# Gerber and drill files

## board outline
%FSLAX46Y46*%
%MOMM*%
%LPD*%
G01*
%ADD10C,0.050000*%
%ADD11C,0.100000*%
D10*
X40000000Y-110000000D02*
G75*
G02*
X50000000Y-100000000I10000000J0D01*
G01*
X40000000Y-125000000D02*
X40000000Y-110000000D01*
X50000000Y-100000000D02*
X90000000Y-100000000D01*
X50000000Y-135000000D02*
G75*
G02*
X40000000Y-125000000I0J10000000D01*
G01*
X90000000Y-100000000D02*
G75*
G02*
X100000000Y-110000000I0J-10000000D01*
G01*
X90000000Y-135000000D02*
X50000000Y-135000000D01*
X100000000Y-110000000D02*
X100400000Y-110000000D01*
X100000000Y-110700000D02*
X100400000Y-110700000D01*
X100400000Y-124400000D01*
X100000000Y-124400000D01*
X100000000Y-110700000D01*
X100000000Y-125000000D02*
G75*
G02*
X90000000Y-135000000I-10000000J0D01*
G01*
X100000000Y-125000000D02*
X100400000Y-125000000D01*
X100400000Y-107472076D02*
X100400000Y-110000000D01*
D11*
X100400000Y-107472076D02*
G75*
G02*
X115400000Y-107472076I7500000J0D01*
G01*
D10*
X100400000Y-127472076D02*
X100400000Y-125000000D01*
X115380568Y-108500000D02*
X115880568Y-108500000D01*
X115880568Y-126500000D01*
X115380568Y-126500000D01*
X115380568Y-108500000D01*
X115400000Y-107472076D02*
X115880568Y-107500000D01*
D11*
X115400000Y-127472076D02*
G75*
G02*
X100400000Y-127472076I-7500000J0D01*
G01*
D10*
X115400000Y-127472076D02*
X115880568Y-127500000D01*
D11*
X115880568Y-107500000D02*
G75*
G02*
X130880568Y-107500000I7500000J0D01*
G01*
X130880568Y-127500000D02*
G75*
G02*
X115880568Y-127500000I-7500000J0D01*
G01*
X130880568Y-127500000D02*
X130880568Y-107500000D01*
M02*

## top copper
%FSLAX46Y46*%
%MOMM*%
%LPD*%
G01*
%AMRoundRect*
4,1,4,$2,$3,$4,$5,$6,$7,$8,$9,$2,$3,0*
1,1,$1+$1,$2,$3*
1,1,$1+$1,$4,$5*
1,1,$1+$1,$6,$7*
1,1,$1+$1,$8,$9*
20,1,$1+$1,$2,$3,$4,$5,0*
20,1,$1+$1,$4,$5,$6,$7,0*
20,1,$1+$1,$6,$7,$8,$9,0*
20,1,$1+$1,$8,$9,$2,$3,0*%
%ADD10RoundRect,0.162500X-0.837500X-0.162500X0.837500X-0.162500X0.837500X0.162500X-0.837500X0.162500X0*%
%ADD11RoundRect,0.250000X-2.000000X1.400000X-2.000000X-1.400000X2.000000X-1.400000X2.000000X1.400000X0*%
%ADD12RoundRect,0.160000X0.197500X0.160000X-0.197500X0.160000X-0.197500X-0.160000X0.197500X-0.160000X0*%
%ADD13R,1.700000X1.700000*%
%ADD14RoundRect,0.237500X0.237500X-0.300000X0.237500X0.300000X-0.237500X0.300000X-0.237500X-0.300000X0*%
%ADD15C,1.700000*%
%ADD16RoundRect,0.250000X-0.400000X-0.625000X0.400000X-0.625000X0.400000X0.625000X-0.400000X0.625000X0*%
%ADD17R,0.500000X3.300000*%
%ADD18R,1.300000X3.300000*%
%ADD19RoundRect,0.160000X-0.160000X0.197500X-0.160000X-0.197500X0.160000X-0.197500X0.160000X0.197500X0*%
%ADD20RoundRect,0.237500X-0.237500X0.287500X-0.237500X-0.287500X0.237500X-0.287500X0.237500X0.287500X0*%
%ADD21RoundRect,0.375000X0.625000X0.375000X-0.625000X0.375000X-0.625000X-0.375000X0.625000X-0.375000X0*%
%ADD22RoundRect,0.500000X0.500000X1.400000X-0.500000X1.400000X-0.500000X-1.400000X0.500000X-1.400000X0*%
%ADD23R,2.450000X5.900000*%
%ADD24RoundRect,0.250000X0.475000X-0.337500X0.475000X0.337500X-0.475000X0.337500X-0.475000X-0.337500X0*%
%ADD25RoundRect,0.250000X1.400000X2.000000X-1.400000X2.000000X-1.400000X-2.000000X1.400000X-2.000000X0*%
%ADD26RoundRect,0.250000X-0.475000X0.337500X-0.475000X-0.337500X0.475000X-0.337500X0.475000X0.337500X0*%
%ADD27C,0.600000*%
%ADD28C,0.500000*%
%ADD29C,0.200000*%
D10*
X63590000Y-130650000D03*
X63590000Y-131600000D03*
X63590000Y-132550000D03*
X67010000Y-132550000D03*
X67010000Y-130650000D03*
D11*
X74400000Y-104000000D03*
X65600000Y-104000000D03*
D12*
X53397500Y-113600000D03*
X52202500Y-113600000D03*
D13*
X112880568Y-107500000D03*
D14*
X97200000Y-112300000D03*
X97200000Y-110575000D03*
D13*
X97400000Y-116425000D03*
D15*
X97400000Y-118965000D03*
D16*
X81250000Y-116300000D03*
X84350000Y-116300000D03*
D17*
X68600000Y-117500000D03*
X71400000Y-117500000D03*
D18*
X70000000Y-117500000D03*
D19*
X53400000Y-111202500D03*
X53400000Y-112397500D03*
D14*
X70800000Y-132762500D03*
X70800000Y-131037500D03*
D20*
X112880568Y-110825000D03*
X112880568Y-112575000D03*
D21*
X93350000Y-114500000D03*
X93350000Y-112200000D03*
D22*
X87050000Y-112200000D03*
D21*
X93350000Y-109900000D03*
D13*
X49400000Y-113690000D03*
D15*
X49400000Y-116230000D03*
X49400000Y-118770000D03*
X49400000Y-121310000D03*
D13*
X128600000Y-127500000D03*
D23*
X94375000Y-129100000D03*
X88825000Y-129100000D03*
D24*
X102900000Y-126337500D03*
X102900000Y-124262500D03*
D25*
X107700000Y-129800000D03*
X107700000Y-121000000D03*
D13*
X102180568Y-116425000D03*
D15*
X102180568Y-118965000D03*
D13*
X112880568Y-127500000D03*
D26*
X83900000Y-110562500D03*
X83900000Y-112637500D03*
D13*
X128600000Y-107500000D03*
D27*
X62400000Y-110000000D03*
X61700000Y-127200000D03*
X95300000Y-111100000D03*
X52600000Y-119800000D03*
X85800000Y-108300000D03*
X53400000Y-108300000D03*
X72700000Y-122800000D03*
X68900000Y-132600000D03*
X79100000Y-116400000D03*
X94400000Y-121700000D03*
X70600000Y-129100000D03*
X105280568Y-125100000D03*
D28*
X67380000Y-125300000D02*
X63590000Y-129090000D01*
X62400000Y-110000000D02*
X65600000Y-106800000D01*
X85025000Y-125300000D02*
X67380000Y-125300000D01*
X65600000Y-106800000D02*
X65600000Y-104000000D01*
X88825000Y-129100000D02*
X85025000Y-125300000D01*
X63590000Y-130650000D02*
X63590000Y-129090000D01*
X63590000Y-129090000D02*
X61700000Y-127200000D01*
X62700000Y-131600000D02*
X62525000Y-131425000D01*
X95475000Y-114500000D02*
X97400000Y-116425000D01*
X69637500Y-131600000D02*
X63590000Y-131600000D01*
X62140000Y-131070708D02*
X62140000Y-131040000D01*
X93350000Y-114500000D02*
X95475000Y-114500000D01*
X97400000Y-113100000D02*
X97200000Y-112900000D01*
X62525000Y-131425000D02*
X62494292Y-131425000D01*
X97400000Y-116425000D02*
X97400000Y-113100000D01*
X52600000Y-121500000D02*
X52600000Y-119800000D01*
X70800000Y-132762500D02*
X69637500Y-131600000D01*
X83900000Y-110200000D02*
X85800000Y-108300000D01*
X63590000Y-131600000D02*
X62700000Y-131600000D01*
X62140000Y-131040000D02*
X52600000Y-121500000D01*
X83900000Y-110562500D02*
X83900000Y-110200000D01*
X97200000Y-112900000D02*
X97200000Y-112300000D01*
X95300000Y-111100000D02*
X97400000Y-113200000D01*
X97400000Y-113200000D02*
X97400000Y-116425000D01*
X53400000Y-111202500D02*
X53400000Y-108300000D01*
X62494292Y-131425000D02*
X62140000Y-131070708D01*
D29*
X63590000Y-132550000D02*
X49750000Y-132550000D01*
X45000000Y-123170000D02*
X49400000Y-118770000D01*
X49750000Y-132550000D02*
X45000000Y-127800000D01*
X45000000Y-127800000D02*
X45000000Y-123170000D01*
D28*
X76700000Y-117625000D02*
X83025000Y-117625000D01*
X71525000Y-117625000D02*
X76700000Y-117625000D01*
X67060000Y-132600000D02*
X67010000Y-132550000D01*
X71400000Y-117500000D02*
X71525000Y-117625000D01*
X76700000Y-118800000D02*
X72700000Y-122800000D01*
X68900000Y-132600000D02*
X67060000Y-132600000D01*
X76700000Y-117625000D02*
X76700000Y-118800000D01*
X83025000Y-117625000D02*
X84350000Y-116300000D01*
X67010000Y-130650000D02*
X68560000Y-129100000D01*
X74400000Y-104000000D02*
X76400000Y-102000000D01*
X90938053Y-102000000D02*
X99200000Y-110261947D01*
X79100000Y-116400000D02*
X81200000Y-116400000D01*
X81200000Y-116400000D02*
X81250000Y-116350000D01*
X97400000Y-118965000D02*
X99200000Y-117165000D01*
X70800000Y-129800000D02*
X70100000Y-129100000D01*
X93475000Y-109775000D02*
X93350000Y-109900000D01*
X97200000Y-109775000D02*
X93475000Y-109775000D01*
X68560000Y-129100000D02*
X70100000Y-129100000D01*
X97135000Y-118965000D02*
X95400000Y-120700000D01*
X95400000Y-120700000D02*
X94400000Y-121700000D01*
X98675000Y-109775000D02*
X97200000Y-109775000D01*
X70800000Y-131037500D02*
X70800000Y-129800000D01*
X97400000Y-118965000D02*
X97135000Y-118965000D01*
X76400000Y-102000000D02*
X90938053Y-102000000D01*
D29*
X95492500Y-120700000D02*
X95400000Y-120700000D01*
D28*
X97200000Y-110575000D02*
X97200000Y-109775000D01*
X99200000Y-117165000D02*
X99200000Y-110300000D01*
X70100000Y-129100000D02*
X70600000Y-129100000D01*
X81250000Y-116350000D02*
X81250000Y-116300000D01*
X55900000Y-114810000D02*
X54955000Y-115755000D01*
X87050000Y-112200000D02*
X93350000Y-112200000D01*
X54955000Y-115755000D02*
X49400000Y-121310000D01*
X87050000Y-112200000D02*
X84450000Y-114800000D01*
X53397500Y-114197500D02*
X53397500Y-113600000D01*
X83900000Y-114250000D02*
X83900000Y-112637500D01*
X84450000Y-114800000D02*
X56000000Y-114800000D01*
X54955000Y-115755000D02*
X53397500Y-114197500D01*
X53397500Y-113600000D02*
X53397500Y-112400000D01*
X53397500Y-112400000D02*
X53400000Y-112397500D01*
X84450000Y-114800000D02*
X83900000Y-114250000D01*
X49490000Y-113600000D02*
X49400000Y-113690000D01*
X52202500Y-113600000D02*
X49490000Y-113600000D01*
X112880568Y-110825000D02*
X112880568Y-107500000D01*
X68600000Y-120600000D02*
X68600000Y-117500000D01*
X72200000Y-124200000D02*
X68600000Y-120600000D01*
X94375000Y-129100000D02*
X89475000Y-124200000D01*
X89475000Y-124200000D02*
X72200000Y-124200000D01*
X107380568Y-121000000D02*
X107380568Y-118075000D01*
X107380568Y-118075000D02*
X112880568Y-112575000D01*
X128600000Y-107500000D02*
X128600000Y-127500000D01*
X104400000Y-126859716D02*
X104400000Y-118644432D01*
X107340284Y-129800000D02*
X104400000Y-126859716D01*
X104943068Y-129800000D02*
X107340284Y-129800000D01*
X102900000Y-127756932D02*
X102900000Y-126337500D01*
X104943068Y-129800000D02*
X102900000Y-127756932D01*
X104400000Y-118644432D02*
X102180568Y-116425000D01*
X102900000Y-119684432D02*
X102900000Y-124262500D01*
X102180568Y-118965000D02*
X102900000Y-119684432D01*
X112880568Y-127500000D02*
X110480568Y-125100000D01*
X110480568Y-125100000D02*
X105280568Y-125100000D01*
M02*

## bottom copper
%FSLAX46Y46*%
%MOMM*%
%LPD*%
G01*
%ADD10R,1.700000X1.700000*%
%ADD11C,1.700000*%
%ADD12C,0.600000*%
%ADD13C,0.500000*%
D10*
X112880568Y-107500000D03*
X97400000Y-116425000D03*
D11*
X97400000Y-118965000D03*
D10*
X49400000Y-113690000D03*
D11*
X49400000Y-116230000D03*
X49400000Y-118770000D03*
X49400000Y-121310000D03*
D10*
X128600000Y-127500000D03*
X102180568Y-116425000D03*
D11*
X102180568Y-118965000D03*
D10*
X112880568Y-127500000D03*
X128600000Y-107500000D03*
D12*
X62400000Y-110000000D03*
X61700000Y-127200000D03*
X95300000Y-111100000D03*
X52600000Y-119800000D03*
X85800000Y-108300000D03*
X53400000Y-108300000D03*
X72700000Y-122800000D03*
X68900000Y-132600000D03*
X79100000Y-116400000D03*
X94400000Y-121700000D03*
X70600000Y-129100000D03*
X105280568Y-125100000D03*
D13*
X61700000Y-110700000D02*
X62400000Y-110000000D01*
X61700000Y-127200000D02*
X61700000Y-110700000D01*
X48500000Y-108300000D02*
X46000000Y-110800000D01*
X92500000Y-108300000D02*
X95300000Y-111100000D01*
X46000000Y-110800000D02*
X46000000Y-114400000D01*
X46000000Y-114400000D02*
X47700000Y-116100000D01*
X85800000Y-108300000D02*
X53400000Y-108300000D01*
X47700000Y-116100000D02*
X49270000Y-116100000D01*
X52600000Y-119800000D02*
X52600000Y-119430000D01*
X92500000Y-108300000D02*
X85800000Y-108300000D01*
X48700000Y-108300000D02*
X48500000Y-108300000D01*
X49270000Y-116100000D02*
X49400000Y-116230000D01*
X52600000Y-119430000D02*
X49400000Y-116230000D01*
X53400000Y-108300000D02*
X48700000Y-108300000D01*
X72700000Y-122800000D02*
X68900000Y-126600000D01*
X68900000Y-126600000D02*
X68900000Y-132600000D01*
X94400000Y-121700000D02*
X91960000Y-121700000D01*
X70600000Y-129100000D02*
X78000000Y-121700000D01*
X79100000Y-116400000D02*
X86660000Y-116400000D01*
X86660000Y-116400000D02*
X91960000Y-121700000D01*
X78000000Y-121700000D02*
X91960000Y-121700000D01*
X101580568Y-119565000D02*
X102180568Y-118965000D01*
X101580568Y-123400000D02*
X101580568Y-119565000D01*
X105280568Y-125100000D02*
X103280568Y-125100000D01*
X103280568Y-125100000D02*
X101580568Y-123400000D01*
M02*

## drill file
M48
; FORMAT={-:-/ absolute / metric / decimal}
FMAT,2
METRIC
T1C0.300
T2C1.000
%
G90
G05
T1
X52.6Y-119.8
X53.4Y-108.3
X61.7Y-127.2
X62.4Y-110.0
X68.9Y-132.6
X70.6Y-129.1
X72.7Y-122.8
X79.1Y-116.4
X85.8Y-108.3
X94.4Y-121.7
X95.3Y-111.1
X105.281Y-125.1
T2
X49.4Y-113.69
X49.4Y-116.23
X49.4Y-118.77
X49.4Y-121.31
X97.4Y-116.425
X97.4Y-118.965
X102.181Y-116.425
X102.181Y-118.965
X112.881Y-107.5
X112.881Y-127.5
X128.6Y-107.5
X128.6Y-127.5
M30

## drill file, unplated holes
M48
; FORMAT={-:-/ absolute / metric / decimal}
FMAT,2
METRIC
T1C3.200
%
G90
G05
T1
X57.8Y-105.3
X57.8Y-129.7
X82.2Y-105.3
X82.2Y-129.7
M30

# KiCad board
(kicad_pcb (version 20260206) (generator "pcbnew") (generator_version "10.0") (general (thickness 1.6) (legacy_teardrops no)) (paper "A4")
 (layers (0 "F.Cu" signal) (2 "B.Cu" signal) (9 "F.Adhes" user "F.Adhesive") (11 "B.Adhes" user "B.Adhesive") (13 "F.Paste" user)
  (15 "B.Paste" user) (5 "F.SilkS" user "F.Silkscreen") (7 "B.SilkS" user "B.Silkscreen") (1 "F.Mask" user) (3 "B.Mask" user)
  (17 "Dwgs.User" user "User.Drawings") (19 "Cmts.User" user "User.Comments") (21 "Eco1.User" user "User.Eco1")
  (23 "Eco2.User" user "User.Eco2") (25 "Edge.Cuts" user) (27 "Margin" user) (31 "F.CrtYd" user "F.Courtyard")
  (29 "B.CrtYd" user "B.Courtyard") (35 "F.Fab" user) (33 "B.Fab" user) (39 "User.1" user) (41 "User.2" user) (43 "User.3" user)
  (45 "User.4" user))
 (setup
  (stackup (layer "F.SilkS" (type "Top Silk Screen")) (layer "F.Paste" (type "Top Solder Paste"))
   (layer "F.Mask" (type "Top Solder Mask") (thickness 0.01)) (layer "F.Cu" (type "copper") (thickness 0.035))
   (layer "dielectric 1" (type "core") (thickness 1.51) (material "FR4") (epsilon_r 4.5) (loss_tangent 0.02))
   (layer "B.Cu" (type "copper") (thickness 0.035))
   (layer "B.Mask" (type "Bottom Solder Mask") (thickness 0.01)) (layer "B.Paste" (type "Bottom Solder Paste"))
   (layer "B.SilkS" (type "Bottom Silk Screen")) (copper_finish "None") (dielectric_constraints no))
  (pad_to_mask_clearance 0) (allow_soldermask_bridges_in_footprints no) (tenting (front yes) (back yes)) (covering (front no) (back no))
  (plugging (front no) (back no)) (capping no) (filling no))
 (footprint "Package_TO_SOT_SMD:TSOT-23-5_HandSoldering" (layer "F.Cu") (at 65.3 131.6)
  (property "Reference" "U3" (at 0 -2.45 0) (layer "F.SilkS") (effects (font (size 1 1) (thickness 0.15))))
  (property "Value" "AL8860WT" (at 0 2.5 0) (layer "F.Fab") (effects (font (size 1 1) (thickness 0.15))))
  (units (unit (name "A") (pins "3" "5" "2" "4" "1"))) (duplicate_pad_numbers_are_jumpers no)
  (pad "1" smd roundrect (at -1.71 -0.95) (size 2 0.65) (layers "F.Cu" "F.Mask" "F.Paste") (roundrect_rratio 0.25) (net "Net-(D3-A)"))
  (pad "2" smd roundrect (at -1.71 0) (size 2 0.65) (layers "F.Cu" "F.Mask" "F.Paste") (roundrect_rratio 0.25) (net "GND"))
  (pad "3" smd roundrect (at -1.71 0.95) (size 2 0.65) (layers "F.Cu" "F.Mask" "F.Paste") (roundrect_rratio 0.25) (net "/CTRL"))
  (pad "4" smd roundrect (at 1.71 0.95) (size 2 0.65) (layers "F.Cu" "F.Mask" "F.Paste") (roundrect_rratio 0.25) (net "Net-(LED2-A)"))
  (pad "5" smd roundrect (at 1.71 -0.95) (size 2 0.65) (layers "F.Cu" "F.Mask" "F.Paste") (roundrect_rratio 0.25) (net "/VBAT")))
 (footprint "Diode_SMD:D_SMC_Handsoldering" (layer "F.Cu") (at 70 104 180)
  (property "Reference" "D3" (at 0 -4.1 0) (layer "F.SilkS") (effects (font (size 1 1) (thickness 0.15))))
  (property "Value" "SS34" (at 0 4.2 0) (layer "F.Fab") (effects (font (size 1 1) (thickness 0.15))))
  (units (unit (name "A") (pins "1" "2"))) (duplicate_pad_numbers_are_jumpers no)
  (pad "1" smd roundrect (at -4.4 0 270) (size 3.3 4.5) (layers "F.Cu" "F.Mask" "F.Paste") (roundrect_rratio 0.0757575758) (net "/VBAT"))
  (pad "2" smd roundrect (at 4.4 0 270) (size 3.3 4.5) (layers "F.Cu" "F.Mask" "F.Paste") (roundrect_rratio 0.0757575758) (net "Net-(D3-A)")))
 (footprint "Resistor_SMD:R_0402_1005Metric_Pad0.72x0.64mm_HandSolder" (layer "F.Cu") (at 52.8 113.6 180)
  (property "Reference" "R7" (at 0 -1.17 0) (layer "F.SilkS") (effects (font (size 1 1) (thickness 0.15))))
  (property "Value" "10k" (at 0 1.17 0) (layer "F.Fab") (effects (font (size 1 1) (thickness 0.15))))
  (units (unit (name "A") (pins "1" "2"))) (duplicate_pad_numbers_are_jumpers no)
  (pad "1" smd roundrect (at -0.5975 0 180) (size 0.715 0.64) (layers "F.Cu" "F.Mask" "F.Paste") (roundrect_rratio 0.25) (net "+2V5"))
  (pad "2" smd roundrect (at 0.5975 0 180) (size 0.715 0.64) (layers "F.Cu" "F.Mask" "F.Paste") (roundrect_rratio 0.25)
   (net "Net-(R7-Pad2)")))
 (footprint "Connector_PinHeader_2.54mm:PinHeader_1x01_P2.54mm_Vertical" (layer "F.Cu") (at 112.880568 107.5)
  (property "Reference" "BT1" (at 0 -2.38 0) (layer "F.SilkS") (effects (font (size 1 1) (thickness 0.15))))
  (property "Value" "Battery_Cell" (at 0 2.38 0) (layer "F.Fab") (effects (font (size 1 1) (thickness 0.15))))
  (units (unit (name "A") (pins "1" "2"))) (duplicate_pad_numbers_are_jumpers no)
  (pad "1" thru_hole rect (at 0 0) (size 1.7 1.7) (drill 1) (layers "*.Cu" "*.Mask") (remove_unused_layers no) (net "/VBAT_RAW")))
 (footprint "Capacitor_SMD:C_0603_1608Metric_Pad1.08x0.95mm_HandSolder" (layer "F.Cu") (at 97.2 111.4375 90)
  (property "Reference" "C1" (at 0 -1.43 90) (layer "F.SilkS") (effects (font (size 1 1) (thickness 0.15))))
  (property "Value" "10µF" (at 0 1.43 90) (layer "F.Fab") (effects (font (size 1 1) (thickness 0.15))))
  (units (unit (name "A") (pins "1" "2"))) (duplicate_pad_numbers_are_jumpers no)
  (pad "1" smd roundrect (at -0.8625 0 90) (size 1.075 0.95) (layers "F.Cu" "F.Mask" "F.Paste") (roundrect_rratio 0.25) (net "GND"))
  (pad "2" smd roundrect (at 0.8625 0 90) (size 1.075 0.95) (layers "F.Cu" "F.Mask" "F.Paste") (roundrect_rratio 0.25) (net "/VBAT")))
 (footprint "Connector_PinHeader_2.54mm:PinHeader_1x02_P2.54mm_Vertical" (layer "F.Cu") (at 97.4 116.425)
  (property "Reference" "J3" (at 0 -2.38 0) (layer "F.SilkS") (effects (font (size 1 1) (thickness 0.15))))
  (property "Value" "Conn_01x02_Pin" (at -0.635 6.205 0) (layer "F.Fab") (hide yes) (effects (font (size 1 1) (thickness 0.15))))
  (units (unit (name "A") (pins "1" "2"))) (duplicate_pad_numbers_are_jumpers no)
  (pad "1" thru_hole rect (at 0 0) (size 1.7 1.7) (drill 1) (layers "*.Cu" "*.Mask") (remove_unused_layers no) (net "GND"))
  (pad "2" thru_hole circle (at 0 2.54) (size 1.7 1.7) (drill 1) (layers "*.Cu" "*.Mask") (remove_unused_layers no) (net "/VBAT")))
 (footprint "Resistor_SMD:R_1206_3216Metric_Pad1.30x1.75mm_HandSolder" (layer "F.Cu") (at 82.8 116.3)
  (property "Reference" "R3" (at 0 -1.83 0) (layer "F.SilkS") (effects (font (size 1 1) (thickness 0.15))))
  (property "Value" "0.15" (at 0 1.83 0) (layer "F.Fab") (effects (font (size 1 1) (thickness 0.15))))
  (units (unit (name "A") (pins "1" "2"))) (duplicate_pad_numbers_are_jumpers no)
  (pad "1" smd roundrect (at -1.55 0) (size 1.3 1.75) (layers "F.Cu" "F.Mask" "F.Paste") (roundrect_rratio 0.192308) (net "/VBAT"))
  (pad "2" smd roundrect (at 1.55 0) (size 1.3 1.75) (layers "F.Cu" "F.Mask" "F.Paste") (roundrect_rratio 0.192308) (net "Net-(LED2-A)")))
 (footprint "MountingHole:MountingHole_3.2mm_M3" (layer "F.Cu") (at 82.2 129.7)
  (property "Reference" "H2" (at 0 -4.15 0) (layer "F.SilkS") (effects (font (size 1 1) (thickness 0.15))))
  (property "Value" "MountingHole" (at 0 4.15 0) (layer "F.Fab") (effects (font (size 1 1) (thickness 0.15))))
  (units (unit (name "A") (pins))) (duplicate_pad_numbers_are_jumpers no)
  (pad "" np_thru_hole circle (at 0 0) (size 3.2 3.2) (drill 3.2) (layers "*.Cu" "*.Mask")))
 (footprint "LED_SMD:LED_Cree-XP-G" (layer "F.Cu") (at 70 117.5)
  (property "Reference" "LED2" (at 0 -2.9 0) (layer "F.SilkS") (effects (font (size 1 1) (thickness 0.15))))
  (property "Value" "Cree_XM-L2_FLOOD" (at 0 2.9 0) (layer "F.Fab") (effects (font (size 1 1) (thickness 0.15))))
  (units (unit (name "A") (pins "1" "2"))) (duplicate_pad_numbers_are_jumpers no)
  (pad "" smd rect (at 0 -1) (size 1.01 0.75) (layers "F.Paste"))
  (pad "" smd rect (at 0 0) (size 1.01 0.75) (layers "F.Paste"))
  (pad "" smd rect (at 0 1) (size 1.01 0.75) (layers "F.Paste"))
  (pad "1" smd rect (at -1.4 0) (size 0.5 3.3) (layers "F.Cu" "F.Mask" "F.Paste") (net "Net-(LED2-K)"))
  (pad "2" smd rect (at 1.4 0) (size 0.5 3.3) (layers "F.Cu" "F.Mask" "F.Paste") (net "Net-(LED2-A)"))
  (pad "3" smd rect (at 0 0) (size 1.3 3.3) (layers "F.Cu" "F.Mask")))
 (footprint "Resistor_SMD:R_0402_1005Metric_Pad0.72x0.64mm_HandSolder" (layer "F.Cu") (at 53.4 111.8 -90)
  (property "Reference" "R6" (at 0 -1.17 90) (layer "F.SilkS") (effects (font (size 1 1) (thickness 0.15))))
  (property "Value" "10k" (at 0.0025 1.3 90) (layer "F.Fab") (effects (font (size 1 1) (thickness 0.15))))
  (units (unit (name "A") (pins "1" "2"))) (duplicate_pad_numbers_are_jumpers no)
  (pad "1" smd roundrect (at -0.5975 0 270) (size 0.715 0.64) (layers "F.Cu" "F.Mask" "F.Paste") (roundrect_rratio 0.25) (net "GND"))
  (pad "2" smd roundrect (at 0.5975 0 270) (size 0.715 0.64) (layers "F.Cu" "F.Mask" "F.Paste") (roundrect_rratio 0.25) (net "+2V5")))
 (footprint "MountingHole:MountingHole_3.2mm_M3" (layer "F.Cu") (at 57.8 129.7)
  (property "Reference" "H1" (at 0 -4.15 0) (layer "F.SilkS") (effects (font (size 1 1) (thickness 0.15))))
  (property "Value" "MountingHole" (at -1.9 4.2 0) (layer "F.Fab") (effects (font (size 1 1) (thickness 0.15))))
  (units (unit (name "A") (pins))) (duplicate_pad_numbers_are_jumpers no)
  (pad "" np_thru_hole circle (at 0 0) (size 3.2 3.2) (drill 3.2) (layers "*.Cu" "*.Mask")))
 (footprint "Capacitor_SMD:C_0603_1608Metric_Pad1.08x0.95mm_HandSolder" (layer "F.Cu") (at 70.8 131.9 90)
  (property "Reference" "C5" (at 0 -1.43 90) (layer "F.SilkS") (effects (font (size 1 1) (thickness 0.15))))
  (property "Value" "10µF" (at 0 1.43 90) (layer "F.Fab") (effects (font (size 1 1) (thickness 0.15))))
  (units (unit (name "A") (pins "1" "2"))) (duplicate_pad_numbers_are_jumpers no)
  (pad "1" smd roundrect (at -0.8625 0 90) (size 1.075 0.95) (layers "F.Cu" "F.Mask" "F.Paste") (roundrect_rratio 0.25) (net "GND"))
  (pad "2" smd roundrect (at 0.8625 0 90) (size 1.075 0.95) (layers "F.Cu" "F.Mask" "F.Paste") (roundrect_rratio 0.25) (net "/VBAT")))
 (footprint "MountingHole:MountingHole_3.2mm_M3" (layer "F.Cu") (at 57.8 105.3)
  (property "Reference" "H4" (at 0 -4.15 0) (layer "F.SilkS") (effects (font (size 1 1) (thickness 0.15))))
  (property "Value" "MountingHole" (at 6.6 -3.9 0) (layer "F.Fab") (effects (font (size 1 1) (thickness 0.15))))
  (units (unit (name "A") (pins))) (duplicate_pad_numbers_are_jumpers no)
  (pad "" np_thru_hole circle (at 0 0) (size 3.2 3.2) (drill 3.2) (layers "*.Cu" "*.Mask")))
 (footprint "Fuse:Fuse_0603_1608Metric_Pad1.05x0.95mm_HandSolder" (layer "F.Cu") (at 112.880568 111.7 -90)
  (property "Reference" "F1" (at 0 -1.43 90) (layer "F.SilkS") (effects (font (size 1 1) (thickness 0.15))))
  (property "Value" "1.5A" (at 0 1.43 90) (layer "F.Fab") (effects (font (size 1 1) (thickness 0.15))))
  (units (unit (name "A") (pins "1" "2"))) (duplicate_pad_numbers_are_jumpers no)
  (pad "1" smd roundrect (at -0.875 0 270) (size 1.05 0.95) (layers "F.Cu" "F.Mask" "F.Paste") (roundrect_rratio 0.25) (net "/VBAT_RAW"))
  (pad "2" smd roundrect (at 0.875 0 270) (size 1.05 0.95) (layers "F.Cu" "F.Mask" "F.Paste") (roundrect_rratio 0.25) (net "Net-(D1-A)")))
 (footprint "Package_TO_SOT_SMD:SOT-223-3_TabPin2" (layer "F.Cu") (at 90.2 112.2 180)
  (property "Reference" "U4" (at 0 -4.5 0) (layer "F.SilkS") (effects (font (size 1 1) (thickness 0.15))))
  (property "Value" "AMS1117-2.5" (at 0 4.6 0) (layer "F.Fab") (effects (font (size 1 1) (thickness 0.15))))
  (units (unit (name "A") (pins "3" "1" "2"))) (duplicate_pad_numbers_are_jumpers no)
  (pad "1" smd roundrect (at -3.15 -2.3 180) (size 2 1.5) (layers "F.Cu" "F.Mask" "F.Paste") (roundrect_rratio 0.25) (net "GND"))
  (pad "2" smd roundrect (at -3.15 0 180) (size 2 1.5) (layers "F.Cu" "F.Mask" "F.Paste") (roundrect_rratio 0.25) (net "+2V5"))
  (pad "2" smd roundrect (at 3.15 0 180) (size 2 3.8) (layers "F.Cu" "F.Mask" "F.Paste") (roundrect_rratio 0.25) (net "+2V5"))
  (pad "3" smd roundrect (at -3.15 2.3 180) (size 2 1.5) (layers "F.Cu" "F.Mask" "F.Paste") (roundrect_rratio 0.25) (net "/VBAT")))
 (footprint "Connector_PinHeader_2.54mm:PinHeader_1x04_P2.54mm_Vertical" (layer "F.Cu") (at 49.4 113.69)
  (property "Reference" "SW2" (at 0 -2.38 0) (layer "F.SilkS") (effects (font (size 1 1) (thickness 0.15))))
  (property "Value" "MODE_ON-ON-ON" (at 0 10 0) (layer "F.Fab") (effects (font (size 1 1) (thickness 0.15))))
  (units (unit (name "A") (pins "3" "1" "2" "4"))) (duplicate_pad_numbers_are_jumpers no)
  (pad "1" thru_hole rect (at 0 0) (size 1.7 1.7) (drill 1) (layers "*.Cu" "*.Mask") (remove_unused_layers no) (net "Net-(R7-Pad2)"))
  (pad "2" thru_hole circle (at 0 2.54) (size 1.7 1.7) (drill 1) (layers "*.Cu" "*.Mask") (remove_unused_layers no) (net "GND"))
  (pad "3" thru_hole circle (at 0 5.08) (size 1.7 1.7) (drill 1) (layers "*.Cu" "*.Mask") (remove_unused_layers no) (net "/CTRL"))
  (pad "4" thru_hole circle (at 0 7.62) (size 1.7 1.7) (drill 1) (layers "*.Cu" "*.Mask") (remove_unused_layers no) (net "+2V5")))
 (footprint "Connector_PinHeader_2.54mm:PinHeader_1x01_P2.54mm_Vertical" (layer "F.Cu") (at 128.6 127.5)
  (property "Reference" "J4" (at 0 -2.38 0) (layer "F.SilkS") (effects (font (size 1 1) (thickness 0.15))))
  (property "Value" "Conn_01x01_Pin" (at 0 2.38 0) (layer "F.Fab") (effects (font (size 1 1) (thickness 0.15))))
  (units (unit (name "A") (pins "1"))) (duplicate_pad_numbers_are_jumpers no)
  (pad "1" thru_hole rect (at 0 0) (size 1.7 1.7) (drill 1) (layers "*.Cu" "*.Mask") (remove_unused_layers no) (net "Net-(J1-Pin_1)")))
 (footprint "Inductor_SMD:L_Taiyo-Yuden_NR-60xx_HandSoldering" (layer "F.Cu") (at 91.6 129.1 180)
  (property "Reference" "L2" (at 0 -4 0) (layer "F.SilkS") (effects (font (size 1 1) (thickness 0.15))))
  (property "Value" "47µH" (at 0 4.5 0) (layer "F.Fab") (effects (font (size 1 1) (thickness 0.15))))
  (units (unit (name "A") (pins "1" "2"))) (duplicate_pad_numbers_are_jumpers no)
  (pad "1" smd rect (at -2.775 0 180) (size 2.45 5.9) (layers "F.Cu" "F.Mask" "F.Paste") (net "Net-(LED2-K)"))
  (pad "2" smd rect (at 2.775 0 180) (size 2.45 5.9) (layers "F.Cu" "F.Mask" "F.Paste") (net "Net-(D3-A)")))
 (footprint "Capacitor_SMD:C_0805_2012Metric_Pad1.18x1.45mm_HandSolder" (layer "F.Cu") (at 102.9 125.3 90)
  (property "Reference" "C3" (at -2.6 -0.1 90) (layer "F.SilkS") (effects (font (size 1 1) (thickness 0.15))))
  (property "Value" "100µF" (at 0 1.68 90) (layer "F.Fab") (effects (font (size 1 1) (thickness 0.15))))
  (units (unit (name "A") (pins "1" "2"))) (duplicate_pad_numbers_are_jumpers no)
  (pad "1" smd roundrect (at -1.0375 0 90) (size 1.175 1.45) (layers "F.Cu" "F.Mask" "F.Paste") (roundrect_rratio 0.212766)
   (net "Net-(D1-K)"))
  (pad "2" smd roundrect (at 1.0375 0 90) (size 1.175 1.45) (layers "F.Cu" "F.Mask" "F.Paste") (roundrect_rratio 0.212766) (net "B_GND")))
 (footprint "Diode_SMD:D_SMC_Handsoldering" (layer "F.Cu") (at 107.7 125.4 90)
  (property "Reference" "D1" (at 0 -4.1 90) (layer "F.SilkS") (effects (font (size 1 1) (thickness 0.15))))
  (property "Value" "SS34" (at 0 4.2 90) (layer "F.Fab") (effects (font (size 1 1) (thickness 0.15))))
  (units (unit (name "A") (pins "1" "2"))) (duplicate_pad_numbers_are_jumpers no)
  (pad "1" smd roundrect (at -4.4 0 180) (size 3.3 4.5) (layers "F.Cu" "F.Mask" "F.Paste") (roundrect_rratio 0.0757575758)
   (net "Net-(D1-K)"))
  (pad "2" smd roundrect (at 4.4 0 180) (size 3.3 4.5) (layers "F.Cu" "F.Mask" "F.Paste") (roundrect_rratio 0.0757575758) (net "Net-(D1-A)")))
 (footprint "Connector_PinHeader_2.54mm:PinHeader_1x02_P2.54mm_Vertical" (layer "F.Cu") (at 102.180568 116.425)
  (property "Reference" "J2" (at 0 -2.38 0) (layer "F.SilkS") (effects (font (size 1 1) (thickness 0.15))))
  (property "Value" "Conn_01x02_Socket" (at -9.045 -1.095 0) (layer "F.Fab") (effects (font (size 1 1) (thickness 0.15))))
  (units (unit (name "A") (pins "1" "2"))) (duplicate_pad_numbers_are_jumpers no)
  (pad "1" thru_hole rect (at 0 0) (size 1.7 1.7) (drill 1) (layers "*.Cu" "*.Mask") (remove_unused_layers no) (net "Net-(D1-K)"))
  (pad "2" thru_hole circle (at 0 2.54) (size 1.7 1.7) (drill 1) (layers "*.Cu" "*.Mask") (remove_unused_layers no) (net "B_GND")))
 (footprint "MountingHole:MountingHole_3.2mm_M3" (layer "F.Cu") (at 82.2 105.3)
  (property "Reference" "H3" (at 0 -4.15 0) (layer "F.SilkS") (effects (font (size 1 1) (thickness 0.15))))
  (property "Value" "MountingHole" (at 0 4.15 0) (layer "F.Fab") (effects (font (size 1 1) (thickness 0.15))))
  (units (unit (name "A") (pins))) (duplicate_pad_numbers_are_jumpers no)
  (pad "" np_thru_hole circle (at 0 0) (size 3.2 3.2) (drill 3.2) (layers "*.Cu" "*.Mask")))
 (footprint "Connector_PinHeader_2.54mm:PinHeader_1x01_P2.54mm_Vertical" (layer "F.Cu") (at 112.880568 127.5)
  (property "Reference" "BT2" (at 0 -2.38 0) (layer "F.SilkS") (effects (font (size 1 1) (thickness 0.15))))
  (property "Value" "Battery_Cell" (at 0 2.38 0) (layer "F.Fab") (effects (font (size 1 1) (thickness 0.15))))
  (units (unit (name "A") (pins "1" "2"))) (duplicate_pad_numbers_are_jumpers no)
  (pad "1" thru_hole rect (at 0 0) (size 1.7 1.7) (drill 1) (layers "*.Cu" "*.Mask") (remove_unused_layers no) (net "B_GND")))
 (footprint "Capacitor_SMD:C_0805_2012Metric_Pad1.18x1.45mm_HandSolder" (layer "F.Cu") (at 83.9 111.6 -90)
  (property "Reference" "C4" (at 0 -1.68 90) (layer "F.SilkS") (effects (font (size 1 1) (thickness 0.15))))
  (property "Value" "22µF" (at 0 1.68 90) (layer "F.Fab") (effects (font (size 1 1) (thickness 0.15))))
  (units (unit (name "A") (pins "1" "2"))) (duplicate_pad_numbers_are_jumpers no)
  (pad "1" smd roundrect (at -1.0375 0 270) (size 1.175 1.45) (layers "F.Cu" "F.Mask" "F.Paste") (roundrect_rratio 0.212766) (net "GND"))
  (pad "2" smd roundrect (at 1.0375 0 270) (size 1.175 1.45) (layers "F.Cu" "F.Mask" "F.Paste") (roundrect_rratio 0.212766) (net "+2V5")))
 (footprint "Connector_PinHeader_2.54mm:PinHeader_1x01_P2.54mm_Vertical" (layer "F.Cu") (at 128.6 107.5)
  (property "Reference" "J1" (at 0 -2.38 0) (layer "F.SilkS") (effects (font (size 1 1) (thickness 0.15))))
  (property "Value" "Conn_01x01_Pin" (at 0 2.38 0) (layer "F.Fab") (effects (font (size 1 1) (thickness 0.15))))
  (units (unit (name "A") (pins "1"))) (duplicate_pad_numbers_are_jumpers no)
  (pad "1" thru_hole rect (at 0 0) (size 1.7 1.7) (drill 1) (layers "*.Cu" "*.Mask") (remove_unused_layers no) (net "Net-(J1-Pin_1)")))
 (gr_arc (start 40 110) (mid 42.928932 102.928932) (end 50 100) (stroke (width 0.05) (type default)) (layer "Edge.Cuts"))
 (gr_line (start 40 125) (end 40 110) (stroke (width 0.05) (type default)) (layer "Edge.Cuts"))
 (gr_line (start 50 100) (end 90 100) (stroke (width 0.05) (type default)) (layer "Edge.Cuts"))
 (gr_arc (start 50 135) (mid 42.928932 132.071068) (end 40 125) (stroke (width 0.05) (type default)) (layer "Edge.Cuts"))
 (gr_arc (start 90 100) (mid 97.071068 102.928932) (end 100 110) (stroke (width 0.05) (type default)) (layer "Edge.Cuts"))
 (gr_line (start 90 135) (end 50 135) (stroke (width 0.05) (type default)) (layer "Edge.Cuts"))
 (gr_line (start 100 110) (end 100.4 110) (stroke (width 0.05) (type default)) (layer "Edge.Cuts"))
 (gr_rect (start 100 110.7) (end 100.4 124.4) (stroke (width 0.05) (type default)) (fill no) (layer "Edge.Cuts"))
 (gr_arc (start 100 125) (mid 97.071068 132.071068) (end 90 135) (stroke (width 0.05) (type default)) (layer "Edge.Cuts"))
 (gr_line (start 100 125) (end 100.4 125) (stroke (width 0.05) (type default)) (layer "Edge.Cuts"))
 (gr_line (start 100.4 107.472076) (end 100.4 110) (stroke (width 0.05) (type default)) (layer "Edge.Cuts"))
 (gr_arc (start 100.4 107.472076) (mid 107.9 99.972076) (end 115.4 107.472076) (stroke (width 0.1) (type solid)) (layer "Edge.Cuts"))
 (gr_line (start 100.4 127.472076) (end 100.4 125) (stroke (width 0.05) (type default)) (layer "Edge.Cuts"))
 (gr_rect (start 115.380568 108.5) (end 115.880568 126.5) (stroke (width 0.05) (type default)) (fill no) (layer "Edge.Cuts"))
 (gr_line (start 115.4 107.472076) (end 115.880568 107.5) (stroke (width 0.05) (type default)) (layer "Edge.Cuts"))
 (gr_arc (start 115.4 127.472076) (mid 107.9 134.972076) (end 100.4 127.472076) (stroke (width 0.1) (type solid)) (layer "Edge.Cuts"))
 (gr_line (start 115.4 127.472076) (end 115.880568 127.5) (stroke (width 0.05) (type default)) (layer "Edge.Cuts"))
 (gr_arc (start 115.880568 107.5) (mid 123.380568 100) (end 130.880568 107.5) (stroke (width 0.1) (type solid)) (layer "Edge.Cuts"))
 (gr_arc (start 130.880568 127.5) (mid 123.380568 135) (end 115.880568 127.5) (stroke (width 0.1) (type solid)) (layer "Edge.Cuts"))
 (gr_line (start 130.880568 127.5) (end 130.880568 107.5) (stroke (width 0.1) (type solid)) (layer "Edge.Cuts"))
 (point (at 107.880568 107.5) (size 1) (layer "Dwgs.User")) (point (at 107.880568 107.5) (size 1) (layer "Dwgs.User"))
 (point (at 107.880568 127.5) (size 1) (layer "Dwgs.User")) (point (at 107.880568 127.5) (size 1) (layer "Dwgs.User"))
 (segment (start 67.38 125.3) (end 63.59 129.09) (width 0.5) (layer "F.Cu") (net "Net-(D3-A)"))
 (segment (start 62.4 110) (end 65.6 106.8) (width 0.5) (layer "F.Cu") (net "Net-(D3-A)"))
 (segment (start 85.025 125.3) (end 67.38 125.3) (width 0.5) (layer "F.Cu") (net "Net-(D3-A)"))
 (segment (start 65.6 106.8) (end 65.6 104) (width 0.5) (layer "F.Cu") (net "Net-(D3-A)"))
 (segment (start 88.825 129.1) (end 85.025 125.3) (width 0.5) (layer "F.Cu") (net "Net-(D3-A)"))
 (segment (start 63.59 130.65) (end 63.59 129.09) (width 0.5) (layer "F.Cu") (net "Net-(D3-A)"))
 (segment (start 63.59 129.09) (end 61.7 127.2) (width 0.5) (layer "F.Cu") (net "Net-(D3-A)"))
 (via (at 62.4 110) (size 0.6) (drill 0.3) (layers "F.Cu" "B.Cu") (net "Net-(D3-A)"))
 (via (at 61.7 127.2) (size 0.6) (drill 0.3) (layers "F.Cu" "B.Cu") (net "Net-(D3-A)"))
 (segment (start 61.7 110.7) (end 62.4 110) (width 0.5) (layer "B.Cu") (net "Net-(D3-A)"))
 (segment (start 61.7 127.2) (end 61.7 110.7) (width 0.5) (layer "B.Cu") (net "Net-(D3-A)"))
 (segment (start 62.7 131.6) (end 62.525 131.425) (width 0.5) (layer "F.Cu") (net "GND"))
 (segment (start 95.475 114.5) (end 97.4 116.425) (width 0.5) (layer "F.Cu") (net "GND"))
 (segment (start 69.6375 131.6) (end 63.59 131.6) (width 0.5) (layer "F.Cu") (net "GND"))
 (segment (start 62.14 131.070708) (end 62.14 131.04) (width 0.5) (layer "F.Cu") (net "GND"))
 (segment (start 93.35 114.5) (end 95.475 114.5) (width 0.5) (layer "F.Cu") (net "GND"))
 (segment (start 97.4 113.1) (end 97.2 112.9) (width 0.5) (layer "F.Cu") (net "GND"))
 (segment (start 62.525 131.425) (end 62.494292 131.425) (width 0.5) (layer "F.Cu") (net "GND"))
 (segment (start 97.4 116.425) (end 97.4 113.1) (width 0.5) (layer "F.Cu") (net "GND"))
 (segment (start 52.6 121.5) (end 52.6 119.8) (width 0.5) (layer "F.Cu") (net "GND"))
 (segment (start 70.8 132.7625) (end 69.6375 131.6) (width 0.5) (layer "F.Cu") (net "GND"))
 (segment (start 83.9 110.2) (end 85.8 108.3) (width 0.5) (layer "F.Cu") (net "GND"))
 (segment (start 63.59 131.6) (end 62.7 131.6) (width 0.5) (layer "F.Cu") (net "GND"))
 (segment (start 62.14 131.04) (end 52.6 121.5) (width 0.5) (layer "F.Cu") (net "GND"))
 (segment (start 83.9 110.5625) (end 83.9 110.2) (width 0.5) (layer "F.Cu") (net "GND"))
 (segment (start 97.2 112.9) (end 97.2 112.3) (width 0.5) (layer "F.Cu") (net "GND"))
 (segment (start 95.3 111.1) (end 97.4 113.2) (width 0.5) (layer "F.Cu") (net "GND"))
 (segment (start 97.4 113.2) (end 97.4 116.425) (width 0.5) (layer "F.Cu") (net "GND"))
 (segment (start 53.4 111.2025) (end 53.4 108.3) (width 0.5) (layer "F.Cu") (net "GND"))
 (segment (start 62.494292 131.425) (end 62.14 131.070708) (width 0.5) (layer "F.Cu") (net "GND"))
 (via (at 95.3 111.1) (size 0.6) (drill 0.3) (layers "F.Cu" "B.Cu") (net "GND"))
 (via (at 52.6 119.8) (size 0.6) (drill 0.3) (layers "F.Cu" "B.Cu") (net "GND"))
 (via (at 85.8 108.3) (size 0.6) (drill 0.3) (layers "F.Cu" "B.Cu") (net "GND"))
 (via (at 53.4 108.3) (size 0.6) (drill 0.3) (layers "F.Cu" "B.Cu") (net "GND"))
 (segment (start 48.5 108.3) (end 46 110.8) (width 0.5) (layer "B.Cu") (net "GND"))
 (segment (start 92.5 108.3) (end 95.3 111.1) (width 0.5) (layer "B.Cu") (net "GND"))
 (segment (start 46 110.8) (end 46 114.4) (width 0.5) (layer "B.Cu") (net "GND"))
 (segment (start 46 114.4) (end 47.7 116.1) (width 0.5) (layer "B.Cu") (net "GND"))
 (segment (start 85.8 108.3) (end 53.4 108.3) (width 0.5) (layer "B.Cu") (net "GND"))
 (segment (start 47.7 116.1) (end 49.27 116.1) (width 0.5) (layer "B.Cu") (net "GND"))
 (segment (start 52.6 119.8) (end 52.6 119.43) (width 0.5) (layer "B.Cu") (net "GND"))
 (segment (start 92.5 108.3) (end 85.8 108.3) (width 0.5) (layer "B.Cu") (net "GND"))
 (segment (start 48.7 108.3) (end 48.5 108.3) (width 0.5) (layer "B.Cu") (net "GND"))
 (segment (start 49.27 116.1) (end 49.4 116.23) (width 0.5) (layer "B.Cu") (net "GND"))
 (segment (start 52.6 119.43) (end 49.4 116.23) (width 0.5) (layer "B.Cu") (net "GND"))
 (segment (start 53.4 108.3) (end 48.7 108.3) (width 0.5) (layer "B.Cu") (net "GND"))
 (segment (start 63.59 132.55) (end 49.75 132.55) (width 0.2) (layer "F.Cu") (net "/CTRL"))
 (segment (start 45 123.17) (end 49.4 118.77) (width 0.2) (layer "F.Cu") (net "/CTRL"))
 (segment (start 49.75 132.55) (end 45 127.8) (width 0.2) (layer "F.Cu") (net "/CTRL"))
 (segment (start 45 127.8) (end 45 123.17) (width 0.2) (layer "F.Cu") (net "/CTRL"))
 (segment (start 76.7 117.625) (end 83.025 117.625) (width 0.5) (layer "F.Cu") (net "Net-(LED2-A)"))
 (segment (start 71.525 117.625) (end 76.7 117.625) (width 0.5) (layer "F.Cu") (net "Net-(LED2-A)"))
 (segment (start 67.06 132.6) (end 67.01 132.55) (width 0.5) (layer "F.Cu") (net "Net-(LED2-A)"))
 (segment (start 71.4 117.5) (end 71.525 117.625) (width 0.5) (layer "F.Cu") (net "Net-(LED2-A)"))
 (segment (start 76.7 118.8) (end 72.7 122.8) (width 0.5) (layer "F.Cu") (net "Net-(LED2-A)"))
 (segment (start 68.9 132.6) (end 67.06 132.6) (width 0.5) (layer "F.Cu") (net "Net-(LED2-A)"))
 (segment (start 76.7 117.625) (end 76.7 118.8) (width 0.5) (layer "F.Cu") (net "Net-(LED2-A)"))
 (segment (start 83.025 117.625) (end 84.35 116.3) (width 0.5) (layer "F.Cu") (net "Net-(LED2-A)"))
 (via (at 72.7 122.8) (size 0.6) (drill 0.3) (layers "F.Cu" "B.Cu") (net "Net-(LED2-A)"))
 (via (at 68.9 132.6) (size 0.6) (drill 0.3) (layers "F.Cu" "B.Cu") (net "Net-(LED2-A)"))
 (segment (start 72.7 122.8) (end 68.9 126.6) (width 0.5) (layer "B.Cu") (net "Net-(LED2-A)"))
 (segment (start 68.9 126.6) (end 68.9 132.6) (width 0.5) (layer "B.Cu") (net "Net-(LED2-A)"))
 (segment (start 67.01 130.65) (end 68.56 129.1) (width 0.5) (layer "F.Cu") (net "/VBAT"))
 (segment (start 74.4 104) (end 76.4 102) (width 0.5) (layer "F.Cu") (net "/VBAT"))
 (segment (start 90.938053 102) (end 99.2 110.261947) (width 0.5) (layer "F.Cu") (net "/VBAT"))
 (segment (start 79.1 116.4) (end 81.2 116.4) (width 0.5) (layer "F.Cu") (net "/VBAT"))
 (segment (start 81.2 116.4) (end 81.25 116.35) (width 0.5) (layer "F.Cu") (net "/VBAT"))
 (segment (start 97.4 118.965) (end 99.2 117.165) (width 0.5) (layer "F.Cu") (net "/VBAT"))
 (segment (start 70.8 129.8) (end 70.1 129.1) (width 0.5) (layer "F.Cu") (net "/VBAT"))
 (segment (start 93.475 109.775) (end 93.35 109.9) (width 0.5) (layer "F.Cu") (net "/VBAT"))
 (segment (start 97.2 109.775) (end 93.475 109.775) (width 0.5) (layer "F.Cu") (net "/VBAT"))
 (segment (start 68.56 129.1) (end 70.1 129.1) (width 0.5) (layer "F.Cu") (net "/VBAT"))
 (segment (start 97.135 118.965) (end 95.4 120.7) (width 0.5) (layer "F.Cu") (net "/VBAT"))
 (segment (start 95.4 120.7) (end 94.4 121.7) (width 0.5) (layer "F.Cu") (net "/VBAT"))
 (segment (start 98.675 109.775) (end 97.2 109.775) (width 0.5) (layer "F.Cu") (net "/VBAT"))
 (segment (start 70.8 131.0375) (end 70.8 129.8) (width 0.5) (layer "F.Cu") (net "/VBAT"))
 (segment (start 97.4 118.965) (end 97.135 118.965) (width 0.5) (layer "F.Cu") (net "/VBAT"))
 (segment (start 76.4 102) (end 90.938053 102) (width 0.5) (layer "F.Cu") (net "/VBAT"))
 (segment (start 95.4925 120.7) (end 95.4 120.7) (width 0.2) (layer "F.Cu") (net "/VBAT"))
 (segment (start 97.2 110.575) (end 97.2 109.775) (width 0.5) (layer "F.Cu") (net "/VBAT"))
 (segment (start 99.2 117.165) (end 99.2 110.3) (width 0.5) (layer "F.Cu") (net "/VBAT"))
 (segment (start 70.1 129.1) (end 70.6 129.1) (width 0.5) (layer "F.Cu") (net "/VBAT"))
 (segment (start 81.25 116.35) (end 81.25 116.3) (width 0.5) (layer "F.Cu") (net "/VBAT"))
 (via (at 79.1 116.4) (size 0.6) (drill 0.3) (layers "F.Cu" "B.Cu") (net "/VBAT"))
 (via (at 94.4 121.7) (size 0.6) (drill 0.3) (layers "F.Cu" "B.Cu") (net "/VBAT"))
 (via (at 70.6 129.1) (size 0.6) (drill 0.3) (layers "F.Cu" "B.Cu") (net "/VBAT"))
 (segment (start 94.4 121.7) (end 91.96 121.7) (width 0.5) (layer "B.Cu") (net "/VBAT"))
 (segment (start 70.6 129.1) (end 78 121.7) (width 0.5) (layer "B.Cu") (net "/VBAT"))
 (segment (start 79.1 116.4) (end 86.66 116.4) (width 0.5) (layer "B.Cu") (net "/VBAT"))
 (segment (start 86.66 116.4) (end 91.96 121.7) (width 0.5) (layer "B.Cu") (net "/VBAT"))
 (segment (start 78 121.7) (end 91.96 121.7) (width 0.5) (layer "B.Cu") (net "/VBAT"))
 (segment (start 55.9 114.81) (end 54.955 115.755) (width 0.5) (layer "F.Cu") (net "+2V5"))
 (segment (start 87.05 112.2) (end 93.35 112.2) (width 0.5) (layer "F.Cu") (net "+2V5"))
 (segment (start 54.955 115.755) (end 49.4 121.31) (width 0.5) (layer "F.Cu") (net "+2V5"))
 (segment (start 87.05 112.2) (end 84.45 114.8) (width 0.5) (layer "F.Cu") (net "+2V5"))
 (segment (start 53.3975 114.1975) (end 53.3975 113.6) (width 0.5) (layer "F.Cu") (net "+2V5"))
 (segment (start 83.9 114.25) (end 83.9 112.6375) (width 0.5) (layer "F.Cu") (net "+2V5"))
 (segment (start 84.45 114.8) (end 56 114.8) (width 0.5) (layer "F.Cu") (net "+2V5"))
 (segment (start 54.955 115.755) (end 53.3975 114.1975) (width 0.5) (layer "F.Cu") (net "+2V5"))
 (segment (start 53.3975 113.6) (end 53.3975 112.4) (width 0.5) (layer "F.Cu") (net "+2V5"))
 (segment (start 53.3975 112.4) (end 53.4 112.3975) (width 0.5) (layer "F.Cu") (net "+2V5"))
 (segment (start 84.45 114.8) (end 83.9 114.25) (width 0.5) (layer "F.Cu") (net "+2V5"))
 (segment (start 49.49 113.6) (end 49.4 113.69) (width 0.5) (layer "F.Cu") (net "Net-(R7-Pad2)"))
 (segment (start 52.2025 113.6) (end 49.49 113.6) (width 0.5) (layer "F.Cu") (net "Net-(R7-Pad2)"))
 (segment (start 112.880568 110.825) (end 112.880568 107.5) (width 0.5) (layer "F.Cu") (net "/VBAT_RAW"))
 (segment (start 68.6 120.6) (end 68.6 117.5) (width 0.5) (layer "F.Cu") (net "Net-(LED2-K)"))
 (segment (start 72.2 124.2) (end 68.6 120.6) (width 0.5) (layer "F.Cu") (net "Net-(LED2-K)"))
 (segment (start 94.375 129.1) (end 89.475 124.2) (width 0.5) (layer "F.Cu") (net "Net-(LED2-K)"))
 (segment (start 89.475 124.2) (end 72.2 124.2) (width 0.5) (layer "F.Cu") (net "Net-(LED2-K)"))
 (segment (start 107.380568 121) (end 107.380568 118.075) (width 0.5) (layer "F.Cu") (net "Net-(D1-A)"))
 (segment (start 107.380568 118.075) (end 112.880568 112.575) (width 0.5) (layer "F.Cu") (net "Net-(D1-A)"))
 (segment (start 128.6 107.5) (end 128.6 127.5) (width 0.5) (layer "F.Cu") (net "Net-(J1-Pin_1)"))
 (segment (start 104.4 126.859716) (end 104.4 118.644432) (width 0.5) (layer "F.Cu") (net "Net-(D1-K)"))
 (segment (start 107.340284 129.8) (end 104.4 126.859716) (width 0.5) (layer "F.Cu") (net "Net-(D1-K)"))
 (segment (start 104.943068 129.8) (end 107.340284 129.8) (width 0.5) (layer "F.Cu") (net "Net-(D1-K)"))
 (segment (start 102.9 127.756932) (end 102.9 126.3375) (width 0.5) (layer "F.Cu") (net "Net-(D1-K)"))
 (segment (start 104.943068 129.8) (end 102.9 127.756932) (width 0.5) (layer "F.Cu") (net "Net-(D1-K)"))
 (segment (start 104.4 118.644432) (end 102.180568 116.425) (width 0.5) (layer "F.Cu") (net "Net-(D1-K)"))
 (segment (start 102.9 119.684432) (end 102.9 124.2625) (width 0.5) (layer "F.Cu") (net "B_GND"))
 (segment (start 102.180568 118.965) (end 102.9 119.684432) (width 0.5) (layer "F.Cu") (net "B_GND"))
 (segment (start 112.880568 127.5) (end 110.480568 125.1) (width 0.5) (layer "F.Cu") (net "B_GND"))
 (segment (start 110.480568 125.1) (end 105.280568 125.1) (width 0.5) (layer "F.Cu") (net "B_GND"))
 (via (at 105.280568 125.1) (size 0.6) (drill 0.3) (layers "F.Cu" "B.Cu") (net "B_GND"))
 (segment (start 101.580568 119.565) (end 102.180568 118.965) (width 0.5) (layer "B.Cu") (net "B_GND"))
 (segment (start 101.580568 123.4) (end 101.580568 119.565) (width 0.5) (layer "B.Cu") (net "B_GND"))
 (segment (start 105.280568 125.1) (end 103.280568 125.1) (width 0.5) (layer "B.Cu") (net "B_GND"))
 (segment (start 103.280568 125.1) (end 101.580568 123.4) (width 0.5) (layer "B.Cu") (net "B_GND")))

